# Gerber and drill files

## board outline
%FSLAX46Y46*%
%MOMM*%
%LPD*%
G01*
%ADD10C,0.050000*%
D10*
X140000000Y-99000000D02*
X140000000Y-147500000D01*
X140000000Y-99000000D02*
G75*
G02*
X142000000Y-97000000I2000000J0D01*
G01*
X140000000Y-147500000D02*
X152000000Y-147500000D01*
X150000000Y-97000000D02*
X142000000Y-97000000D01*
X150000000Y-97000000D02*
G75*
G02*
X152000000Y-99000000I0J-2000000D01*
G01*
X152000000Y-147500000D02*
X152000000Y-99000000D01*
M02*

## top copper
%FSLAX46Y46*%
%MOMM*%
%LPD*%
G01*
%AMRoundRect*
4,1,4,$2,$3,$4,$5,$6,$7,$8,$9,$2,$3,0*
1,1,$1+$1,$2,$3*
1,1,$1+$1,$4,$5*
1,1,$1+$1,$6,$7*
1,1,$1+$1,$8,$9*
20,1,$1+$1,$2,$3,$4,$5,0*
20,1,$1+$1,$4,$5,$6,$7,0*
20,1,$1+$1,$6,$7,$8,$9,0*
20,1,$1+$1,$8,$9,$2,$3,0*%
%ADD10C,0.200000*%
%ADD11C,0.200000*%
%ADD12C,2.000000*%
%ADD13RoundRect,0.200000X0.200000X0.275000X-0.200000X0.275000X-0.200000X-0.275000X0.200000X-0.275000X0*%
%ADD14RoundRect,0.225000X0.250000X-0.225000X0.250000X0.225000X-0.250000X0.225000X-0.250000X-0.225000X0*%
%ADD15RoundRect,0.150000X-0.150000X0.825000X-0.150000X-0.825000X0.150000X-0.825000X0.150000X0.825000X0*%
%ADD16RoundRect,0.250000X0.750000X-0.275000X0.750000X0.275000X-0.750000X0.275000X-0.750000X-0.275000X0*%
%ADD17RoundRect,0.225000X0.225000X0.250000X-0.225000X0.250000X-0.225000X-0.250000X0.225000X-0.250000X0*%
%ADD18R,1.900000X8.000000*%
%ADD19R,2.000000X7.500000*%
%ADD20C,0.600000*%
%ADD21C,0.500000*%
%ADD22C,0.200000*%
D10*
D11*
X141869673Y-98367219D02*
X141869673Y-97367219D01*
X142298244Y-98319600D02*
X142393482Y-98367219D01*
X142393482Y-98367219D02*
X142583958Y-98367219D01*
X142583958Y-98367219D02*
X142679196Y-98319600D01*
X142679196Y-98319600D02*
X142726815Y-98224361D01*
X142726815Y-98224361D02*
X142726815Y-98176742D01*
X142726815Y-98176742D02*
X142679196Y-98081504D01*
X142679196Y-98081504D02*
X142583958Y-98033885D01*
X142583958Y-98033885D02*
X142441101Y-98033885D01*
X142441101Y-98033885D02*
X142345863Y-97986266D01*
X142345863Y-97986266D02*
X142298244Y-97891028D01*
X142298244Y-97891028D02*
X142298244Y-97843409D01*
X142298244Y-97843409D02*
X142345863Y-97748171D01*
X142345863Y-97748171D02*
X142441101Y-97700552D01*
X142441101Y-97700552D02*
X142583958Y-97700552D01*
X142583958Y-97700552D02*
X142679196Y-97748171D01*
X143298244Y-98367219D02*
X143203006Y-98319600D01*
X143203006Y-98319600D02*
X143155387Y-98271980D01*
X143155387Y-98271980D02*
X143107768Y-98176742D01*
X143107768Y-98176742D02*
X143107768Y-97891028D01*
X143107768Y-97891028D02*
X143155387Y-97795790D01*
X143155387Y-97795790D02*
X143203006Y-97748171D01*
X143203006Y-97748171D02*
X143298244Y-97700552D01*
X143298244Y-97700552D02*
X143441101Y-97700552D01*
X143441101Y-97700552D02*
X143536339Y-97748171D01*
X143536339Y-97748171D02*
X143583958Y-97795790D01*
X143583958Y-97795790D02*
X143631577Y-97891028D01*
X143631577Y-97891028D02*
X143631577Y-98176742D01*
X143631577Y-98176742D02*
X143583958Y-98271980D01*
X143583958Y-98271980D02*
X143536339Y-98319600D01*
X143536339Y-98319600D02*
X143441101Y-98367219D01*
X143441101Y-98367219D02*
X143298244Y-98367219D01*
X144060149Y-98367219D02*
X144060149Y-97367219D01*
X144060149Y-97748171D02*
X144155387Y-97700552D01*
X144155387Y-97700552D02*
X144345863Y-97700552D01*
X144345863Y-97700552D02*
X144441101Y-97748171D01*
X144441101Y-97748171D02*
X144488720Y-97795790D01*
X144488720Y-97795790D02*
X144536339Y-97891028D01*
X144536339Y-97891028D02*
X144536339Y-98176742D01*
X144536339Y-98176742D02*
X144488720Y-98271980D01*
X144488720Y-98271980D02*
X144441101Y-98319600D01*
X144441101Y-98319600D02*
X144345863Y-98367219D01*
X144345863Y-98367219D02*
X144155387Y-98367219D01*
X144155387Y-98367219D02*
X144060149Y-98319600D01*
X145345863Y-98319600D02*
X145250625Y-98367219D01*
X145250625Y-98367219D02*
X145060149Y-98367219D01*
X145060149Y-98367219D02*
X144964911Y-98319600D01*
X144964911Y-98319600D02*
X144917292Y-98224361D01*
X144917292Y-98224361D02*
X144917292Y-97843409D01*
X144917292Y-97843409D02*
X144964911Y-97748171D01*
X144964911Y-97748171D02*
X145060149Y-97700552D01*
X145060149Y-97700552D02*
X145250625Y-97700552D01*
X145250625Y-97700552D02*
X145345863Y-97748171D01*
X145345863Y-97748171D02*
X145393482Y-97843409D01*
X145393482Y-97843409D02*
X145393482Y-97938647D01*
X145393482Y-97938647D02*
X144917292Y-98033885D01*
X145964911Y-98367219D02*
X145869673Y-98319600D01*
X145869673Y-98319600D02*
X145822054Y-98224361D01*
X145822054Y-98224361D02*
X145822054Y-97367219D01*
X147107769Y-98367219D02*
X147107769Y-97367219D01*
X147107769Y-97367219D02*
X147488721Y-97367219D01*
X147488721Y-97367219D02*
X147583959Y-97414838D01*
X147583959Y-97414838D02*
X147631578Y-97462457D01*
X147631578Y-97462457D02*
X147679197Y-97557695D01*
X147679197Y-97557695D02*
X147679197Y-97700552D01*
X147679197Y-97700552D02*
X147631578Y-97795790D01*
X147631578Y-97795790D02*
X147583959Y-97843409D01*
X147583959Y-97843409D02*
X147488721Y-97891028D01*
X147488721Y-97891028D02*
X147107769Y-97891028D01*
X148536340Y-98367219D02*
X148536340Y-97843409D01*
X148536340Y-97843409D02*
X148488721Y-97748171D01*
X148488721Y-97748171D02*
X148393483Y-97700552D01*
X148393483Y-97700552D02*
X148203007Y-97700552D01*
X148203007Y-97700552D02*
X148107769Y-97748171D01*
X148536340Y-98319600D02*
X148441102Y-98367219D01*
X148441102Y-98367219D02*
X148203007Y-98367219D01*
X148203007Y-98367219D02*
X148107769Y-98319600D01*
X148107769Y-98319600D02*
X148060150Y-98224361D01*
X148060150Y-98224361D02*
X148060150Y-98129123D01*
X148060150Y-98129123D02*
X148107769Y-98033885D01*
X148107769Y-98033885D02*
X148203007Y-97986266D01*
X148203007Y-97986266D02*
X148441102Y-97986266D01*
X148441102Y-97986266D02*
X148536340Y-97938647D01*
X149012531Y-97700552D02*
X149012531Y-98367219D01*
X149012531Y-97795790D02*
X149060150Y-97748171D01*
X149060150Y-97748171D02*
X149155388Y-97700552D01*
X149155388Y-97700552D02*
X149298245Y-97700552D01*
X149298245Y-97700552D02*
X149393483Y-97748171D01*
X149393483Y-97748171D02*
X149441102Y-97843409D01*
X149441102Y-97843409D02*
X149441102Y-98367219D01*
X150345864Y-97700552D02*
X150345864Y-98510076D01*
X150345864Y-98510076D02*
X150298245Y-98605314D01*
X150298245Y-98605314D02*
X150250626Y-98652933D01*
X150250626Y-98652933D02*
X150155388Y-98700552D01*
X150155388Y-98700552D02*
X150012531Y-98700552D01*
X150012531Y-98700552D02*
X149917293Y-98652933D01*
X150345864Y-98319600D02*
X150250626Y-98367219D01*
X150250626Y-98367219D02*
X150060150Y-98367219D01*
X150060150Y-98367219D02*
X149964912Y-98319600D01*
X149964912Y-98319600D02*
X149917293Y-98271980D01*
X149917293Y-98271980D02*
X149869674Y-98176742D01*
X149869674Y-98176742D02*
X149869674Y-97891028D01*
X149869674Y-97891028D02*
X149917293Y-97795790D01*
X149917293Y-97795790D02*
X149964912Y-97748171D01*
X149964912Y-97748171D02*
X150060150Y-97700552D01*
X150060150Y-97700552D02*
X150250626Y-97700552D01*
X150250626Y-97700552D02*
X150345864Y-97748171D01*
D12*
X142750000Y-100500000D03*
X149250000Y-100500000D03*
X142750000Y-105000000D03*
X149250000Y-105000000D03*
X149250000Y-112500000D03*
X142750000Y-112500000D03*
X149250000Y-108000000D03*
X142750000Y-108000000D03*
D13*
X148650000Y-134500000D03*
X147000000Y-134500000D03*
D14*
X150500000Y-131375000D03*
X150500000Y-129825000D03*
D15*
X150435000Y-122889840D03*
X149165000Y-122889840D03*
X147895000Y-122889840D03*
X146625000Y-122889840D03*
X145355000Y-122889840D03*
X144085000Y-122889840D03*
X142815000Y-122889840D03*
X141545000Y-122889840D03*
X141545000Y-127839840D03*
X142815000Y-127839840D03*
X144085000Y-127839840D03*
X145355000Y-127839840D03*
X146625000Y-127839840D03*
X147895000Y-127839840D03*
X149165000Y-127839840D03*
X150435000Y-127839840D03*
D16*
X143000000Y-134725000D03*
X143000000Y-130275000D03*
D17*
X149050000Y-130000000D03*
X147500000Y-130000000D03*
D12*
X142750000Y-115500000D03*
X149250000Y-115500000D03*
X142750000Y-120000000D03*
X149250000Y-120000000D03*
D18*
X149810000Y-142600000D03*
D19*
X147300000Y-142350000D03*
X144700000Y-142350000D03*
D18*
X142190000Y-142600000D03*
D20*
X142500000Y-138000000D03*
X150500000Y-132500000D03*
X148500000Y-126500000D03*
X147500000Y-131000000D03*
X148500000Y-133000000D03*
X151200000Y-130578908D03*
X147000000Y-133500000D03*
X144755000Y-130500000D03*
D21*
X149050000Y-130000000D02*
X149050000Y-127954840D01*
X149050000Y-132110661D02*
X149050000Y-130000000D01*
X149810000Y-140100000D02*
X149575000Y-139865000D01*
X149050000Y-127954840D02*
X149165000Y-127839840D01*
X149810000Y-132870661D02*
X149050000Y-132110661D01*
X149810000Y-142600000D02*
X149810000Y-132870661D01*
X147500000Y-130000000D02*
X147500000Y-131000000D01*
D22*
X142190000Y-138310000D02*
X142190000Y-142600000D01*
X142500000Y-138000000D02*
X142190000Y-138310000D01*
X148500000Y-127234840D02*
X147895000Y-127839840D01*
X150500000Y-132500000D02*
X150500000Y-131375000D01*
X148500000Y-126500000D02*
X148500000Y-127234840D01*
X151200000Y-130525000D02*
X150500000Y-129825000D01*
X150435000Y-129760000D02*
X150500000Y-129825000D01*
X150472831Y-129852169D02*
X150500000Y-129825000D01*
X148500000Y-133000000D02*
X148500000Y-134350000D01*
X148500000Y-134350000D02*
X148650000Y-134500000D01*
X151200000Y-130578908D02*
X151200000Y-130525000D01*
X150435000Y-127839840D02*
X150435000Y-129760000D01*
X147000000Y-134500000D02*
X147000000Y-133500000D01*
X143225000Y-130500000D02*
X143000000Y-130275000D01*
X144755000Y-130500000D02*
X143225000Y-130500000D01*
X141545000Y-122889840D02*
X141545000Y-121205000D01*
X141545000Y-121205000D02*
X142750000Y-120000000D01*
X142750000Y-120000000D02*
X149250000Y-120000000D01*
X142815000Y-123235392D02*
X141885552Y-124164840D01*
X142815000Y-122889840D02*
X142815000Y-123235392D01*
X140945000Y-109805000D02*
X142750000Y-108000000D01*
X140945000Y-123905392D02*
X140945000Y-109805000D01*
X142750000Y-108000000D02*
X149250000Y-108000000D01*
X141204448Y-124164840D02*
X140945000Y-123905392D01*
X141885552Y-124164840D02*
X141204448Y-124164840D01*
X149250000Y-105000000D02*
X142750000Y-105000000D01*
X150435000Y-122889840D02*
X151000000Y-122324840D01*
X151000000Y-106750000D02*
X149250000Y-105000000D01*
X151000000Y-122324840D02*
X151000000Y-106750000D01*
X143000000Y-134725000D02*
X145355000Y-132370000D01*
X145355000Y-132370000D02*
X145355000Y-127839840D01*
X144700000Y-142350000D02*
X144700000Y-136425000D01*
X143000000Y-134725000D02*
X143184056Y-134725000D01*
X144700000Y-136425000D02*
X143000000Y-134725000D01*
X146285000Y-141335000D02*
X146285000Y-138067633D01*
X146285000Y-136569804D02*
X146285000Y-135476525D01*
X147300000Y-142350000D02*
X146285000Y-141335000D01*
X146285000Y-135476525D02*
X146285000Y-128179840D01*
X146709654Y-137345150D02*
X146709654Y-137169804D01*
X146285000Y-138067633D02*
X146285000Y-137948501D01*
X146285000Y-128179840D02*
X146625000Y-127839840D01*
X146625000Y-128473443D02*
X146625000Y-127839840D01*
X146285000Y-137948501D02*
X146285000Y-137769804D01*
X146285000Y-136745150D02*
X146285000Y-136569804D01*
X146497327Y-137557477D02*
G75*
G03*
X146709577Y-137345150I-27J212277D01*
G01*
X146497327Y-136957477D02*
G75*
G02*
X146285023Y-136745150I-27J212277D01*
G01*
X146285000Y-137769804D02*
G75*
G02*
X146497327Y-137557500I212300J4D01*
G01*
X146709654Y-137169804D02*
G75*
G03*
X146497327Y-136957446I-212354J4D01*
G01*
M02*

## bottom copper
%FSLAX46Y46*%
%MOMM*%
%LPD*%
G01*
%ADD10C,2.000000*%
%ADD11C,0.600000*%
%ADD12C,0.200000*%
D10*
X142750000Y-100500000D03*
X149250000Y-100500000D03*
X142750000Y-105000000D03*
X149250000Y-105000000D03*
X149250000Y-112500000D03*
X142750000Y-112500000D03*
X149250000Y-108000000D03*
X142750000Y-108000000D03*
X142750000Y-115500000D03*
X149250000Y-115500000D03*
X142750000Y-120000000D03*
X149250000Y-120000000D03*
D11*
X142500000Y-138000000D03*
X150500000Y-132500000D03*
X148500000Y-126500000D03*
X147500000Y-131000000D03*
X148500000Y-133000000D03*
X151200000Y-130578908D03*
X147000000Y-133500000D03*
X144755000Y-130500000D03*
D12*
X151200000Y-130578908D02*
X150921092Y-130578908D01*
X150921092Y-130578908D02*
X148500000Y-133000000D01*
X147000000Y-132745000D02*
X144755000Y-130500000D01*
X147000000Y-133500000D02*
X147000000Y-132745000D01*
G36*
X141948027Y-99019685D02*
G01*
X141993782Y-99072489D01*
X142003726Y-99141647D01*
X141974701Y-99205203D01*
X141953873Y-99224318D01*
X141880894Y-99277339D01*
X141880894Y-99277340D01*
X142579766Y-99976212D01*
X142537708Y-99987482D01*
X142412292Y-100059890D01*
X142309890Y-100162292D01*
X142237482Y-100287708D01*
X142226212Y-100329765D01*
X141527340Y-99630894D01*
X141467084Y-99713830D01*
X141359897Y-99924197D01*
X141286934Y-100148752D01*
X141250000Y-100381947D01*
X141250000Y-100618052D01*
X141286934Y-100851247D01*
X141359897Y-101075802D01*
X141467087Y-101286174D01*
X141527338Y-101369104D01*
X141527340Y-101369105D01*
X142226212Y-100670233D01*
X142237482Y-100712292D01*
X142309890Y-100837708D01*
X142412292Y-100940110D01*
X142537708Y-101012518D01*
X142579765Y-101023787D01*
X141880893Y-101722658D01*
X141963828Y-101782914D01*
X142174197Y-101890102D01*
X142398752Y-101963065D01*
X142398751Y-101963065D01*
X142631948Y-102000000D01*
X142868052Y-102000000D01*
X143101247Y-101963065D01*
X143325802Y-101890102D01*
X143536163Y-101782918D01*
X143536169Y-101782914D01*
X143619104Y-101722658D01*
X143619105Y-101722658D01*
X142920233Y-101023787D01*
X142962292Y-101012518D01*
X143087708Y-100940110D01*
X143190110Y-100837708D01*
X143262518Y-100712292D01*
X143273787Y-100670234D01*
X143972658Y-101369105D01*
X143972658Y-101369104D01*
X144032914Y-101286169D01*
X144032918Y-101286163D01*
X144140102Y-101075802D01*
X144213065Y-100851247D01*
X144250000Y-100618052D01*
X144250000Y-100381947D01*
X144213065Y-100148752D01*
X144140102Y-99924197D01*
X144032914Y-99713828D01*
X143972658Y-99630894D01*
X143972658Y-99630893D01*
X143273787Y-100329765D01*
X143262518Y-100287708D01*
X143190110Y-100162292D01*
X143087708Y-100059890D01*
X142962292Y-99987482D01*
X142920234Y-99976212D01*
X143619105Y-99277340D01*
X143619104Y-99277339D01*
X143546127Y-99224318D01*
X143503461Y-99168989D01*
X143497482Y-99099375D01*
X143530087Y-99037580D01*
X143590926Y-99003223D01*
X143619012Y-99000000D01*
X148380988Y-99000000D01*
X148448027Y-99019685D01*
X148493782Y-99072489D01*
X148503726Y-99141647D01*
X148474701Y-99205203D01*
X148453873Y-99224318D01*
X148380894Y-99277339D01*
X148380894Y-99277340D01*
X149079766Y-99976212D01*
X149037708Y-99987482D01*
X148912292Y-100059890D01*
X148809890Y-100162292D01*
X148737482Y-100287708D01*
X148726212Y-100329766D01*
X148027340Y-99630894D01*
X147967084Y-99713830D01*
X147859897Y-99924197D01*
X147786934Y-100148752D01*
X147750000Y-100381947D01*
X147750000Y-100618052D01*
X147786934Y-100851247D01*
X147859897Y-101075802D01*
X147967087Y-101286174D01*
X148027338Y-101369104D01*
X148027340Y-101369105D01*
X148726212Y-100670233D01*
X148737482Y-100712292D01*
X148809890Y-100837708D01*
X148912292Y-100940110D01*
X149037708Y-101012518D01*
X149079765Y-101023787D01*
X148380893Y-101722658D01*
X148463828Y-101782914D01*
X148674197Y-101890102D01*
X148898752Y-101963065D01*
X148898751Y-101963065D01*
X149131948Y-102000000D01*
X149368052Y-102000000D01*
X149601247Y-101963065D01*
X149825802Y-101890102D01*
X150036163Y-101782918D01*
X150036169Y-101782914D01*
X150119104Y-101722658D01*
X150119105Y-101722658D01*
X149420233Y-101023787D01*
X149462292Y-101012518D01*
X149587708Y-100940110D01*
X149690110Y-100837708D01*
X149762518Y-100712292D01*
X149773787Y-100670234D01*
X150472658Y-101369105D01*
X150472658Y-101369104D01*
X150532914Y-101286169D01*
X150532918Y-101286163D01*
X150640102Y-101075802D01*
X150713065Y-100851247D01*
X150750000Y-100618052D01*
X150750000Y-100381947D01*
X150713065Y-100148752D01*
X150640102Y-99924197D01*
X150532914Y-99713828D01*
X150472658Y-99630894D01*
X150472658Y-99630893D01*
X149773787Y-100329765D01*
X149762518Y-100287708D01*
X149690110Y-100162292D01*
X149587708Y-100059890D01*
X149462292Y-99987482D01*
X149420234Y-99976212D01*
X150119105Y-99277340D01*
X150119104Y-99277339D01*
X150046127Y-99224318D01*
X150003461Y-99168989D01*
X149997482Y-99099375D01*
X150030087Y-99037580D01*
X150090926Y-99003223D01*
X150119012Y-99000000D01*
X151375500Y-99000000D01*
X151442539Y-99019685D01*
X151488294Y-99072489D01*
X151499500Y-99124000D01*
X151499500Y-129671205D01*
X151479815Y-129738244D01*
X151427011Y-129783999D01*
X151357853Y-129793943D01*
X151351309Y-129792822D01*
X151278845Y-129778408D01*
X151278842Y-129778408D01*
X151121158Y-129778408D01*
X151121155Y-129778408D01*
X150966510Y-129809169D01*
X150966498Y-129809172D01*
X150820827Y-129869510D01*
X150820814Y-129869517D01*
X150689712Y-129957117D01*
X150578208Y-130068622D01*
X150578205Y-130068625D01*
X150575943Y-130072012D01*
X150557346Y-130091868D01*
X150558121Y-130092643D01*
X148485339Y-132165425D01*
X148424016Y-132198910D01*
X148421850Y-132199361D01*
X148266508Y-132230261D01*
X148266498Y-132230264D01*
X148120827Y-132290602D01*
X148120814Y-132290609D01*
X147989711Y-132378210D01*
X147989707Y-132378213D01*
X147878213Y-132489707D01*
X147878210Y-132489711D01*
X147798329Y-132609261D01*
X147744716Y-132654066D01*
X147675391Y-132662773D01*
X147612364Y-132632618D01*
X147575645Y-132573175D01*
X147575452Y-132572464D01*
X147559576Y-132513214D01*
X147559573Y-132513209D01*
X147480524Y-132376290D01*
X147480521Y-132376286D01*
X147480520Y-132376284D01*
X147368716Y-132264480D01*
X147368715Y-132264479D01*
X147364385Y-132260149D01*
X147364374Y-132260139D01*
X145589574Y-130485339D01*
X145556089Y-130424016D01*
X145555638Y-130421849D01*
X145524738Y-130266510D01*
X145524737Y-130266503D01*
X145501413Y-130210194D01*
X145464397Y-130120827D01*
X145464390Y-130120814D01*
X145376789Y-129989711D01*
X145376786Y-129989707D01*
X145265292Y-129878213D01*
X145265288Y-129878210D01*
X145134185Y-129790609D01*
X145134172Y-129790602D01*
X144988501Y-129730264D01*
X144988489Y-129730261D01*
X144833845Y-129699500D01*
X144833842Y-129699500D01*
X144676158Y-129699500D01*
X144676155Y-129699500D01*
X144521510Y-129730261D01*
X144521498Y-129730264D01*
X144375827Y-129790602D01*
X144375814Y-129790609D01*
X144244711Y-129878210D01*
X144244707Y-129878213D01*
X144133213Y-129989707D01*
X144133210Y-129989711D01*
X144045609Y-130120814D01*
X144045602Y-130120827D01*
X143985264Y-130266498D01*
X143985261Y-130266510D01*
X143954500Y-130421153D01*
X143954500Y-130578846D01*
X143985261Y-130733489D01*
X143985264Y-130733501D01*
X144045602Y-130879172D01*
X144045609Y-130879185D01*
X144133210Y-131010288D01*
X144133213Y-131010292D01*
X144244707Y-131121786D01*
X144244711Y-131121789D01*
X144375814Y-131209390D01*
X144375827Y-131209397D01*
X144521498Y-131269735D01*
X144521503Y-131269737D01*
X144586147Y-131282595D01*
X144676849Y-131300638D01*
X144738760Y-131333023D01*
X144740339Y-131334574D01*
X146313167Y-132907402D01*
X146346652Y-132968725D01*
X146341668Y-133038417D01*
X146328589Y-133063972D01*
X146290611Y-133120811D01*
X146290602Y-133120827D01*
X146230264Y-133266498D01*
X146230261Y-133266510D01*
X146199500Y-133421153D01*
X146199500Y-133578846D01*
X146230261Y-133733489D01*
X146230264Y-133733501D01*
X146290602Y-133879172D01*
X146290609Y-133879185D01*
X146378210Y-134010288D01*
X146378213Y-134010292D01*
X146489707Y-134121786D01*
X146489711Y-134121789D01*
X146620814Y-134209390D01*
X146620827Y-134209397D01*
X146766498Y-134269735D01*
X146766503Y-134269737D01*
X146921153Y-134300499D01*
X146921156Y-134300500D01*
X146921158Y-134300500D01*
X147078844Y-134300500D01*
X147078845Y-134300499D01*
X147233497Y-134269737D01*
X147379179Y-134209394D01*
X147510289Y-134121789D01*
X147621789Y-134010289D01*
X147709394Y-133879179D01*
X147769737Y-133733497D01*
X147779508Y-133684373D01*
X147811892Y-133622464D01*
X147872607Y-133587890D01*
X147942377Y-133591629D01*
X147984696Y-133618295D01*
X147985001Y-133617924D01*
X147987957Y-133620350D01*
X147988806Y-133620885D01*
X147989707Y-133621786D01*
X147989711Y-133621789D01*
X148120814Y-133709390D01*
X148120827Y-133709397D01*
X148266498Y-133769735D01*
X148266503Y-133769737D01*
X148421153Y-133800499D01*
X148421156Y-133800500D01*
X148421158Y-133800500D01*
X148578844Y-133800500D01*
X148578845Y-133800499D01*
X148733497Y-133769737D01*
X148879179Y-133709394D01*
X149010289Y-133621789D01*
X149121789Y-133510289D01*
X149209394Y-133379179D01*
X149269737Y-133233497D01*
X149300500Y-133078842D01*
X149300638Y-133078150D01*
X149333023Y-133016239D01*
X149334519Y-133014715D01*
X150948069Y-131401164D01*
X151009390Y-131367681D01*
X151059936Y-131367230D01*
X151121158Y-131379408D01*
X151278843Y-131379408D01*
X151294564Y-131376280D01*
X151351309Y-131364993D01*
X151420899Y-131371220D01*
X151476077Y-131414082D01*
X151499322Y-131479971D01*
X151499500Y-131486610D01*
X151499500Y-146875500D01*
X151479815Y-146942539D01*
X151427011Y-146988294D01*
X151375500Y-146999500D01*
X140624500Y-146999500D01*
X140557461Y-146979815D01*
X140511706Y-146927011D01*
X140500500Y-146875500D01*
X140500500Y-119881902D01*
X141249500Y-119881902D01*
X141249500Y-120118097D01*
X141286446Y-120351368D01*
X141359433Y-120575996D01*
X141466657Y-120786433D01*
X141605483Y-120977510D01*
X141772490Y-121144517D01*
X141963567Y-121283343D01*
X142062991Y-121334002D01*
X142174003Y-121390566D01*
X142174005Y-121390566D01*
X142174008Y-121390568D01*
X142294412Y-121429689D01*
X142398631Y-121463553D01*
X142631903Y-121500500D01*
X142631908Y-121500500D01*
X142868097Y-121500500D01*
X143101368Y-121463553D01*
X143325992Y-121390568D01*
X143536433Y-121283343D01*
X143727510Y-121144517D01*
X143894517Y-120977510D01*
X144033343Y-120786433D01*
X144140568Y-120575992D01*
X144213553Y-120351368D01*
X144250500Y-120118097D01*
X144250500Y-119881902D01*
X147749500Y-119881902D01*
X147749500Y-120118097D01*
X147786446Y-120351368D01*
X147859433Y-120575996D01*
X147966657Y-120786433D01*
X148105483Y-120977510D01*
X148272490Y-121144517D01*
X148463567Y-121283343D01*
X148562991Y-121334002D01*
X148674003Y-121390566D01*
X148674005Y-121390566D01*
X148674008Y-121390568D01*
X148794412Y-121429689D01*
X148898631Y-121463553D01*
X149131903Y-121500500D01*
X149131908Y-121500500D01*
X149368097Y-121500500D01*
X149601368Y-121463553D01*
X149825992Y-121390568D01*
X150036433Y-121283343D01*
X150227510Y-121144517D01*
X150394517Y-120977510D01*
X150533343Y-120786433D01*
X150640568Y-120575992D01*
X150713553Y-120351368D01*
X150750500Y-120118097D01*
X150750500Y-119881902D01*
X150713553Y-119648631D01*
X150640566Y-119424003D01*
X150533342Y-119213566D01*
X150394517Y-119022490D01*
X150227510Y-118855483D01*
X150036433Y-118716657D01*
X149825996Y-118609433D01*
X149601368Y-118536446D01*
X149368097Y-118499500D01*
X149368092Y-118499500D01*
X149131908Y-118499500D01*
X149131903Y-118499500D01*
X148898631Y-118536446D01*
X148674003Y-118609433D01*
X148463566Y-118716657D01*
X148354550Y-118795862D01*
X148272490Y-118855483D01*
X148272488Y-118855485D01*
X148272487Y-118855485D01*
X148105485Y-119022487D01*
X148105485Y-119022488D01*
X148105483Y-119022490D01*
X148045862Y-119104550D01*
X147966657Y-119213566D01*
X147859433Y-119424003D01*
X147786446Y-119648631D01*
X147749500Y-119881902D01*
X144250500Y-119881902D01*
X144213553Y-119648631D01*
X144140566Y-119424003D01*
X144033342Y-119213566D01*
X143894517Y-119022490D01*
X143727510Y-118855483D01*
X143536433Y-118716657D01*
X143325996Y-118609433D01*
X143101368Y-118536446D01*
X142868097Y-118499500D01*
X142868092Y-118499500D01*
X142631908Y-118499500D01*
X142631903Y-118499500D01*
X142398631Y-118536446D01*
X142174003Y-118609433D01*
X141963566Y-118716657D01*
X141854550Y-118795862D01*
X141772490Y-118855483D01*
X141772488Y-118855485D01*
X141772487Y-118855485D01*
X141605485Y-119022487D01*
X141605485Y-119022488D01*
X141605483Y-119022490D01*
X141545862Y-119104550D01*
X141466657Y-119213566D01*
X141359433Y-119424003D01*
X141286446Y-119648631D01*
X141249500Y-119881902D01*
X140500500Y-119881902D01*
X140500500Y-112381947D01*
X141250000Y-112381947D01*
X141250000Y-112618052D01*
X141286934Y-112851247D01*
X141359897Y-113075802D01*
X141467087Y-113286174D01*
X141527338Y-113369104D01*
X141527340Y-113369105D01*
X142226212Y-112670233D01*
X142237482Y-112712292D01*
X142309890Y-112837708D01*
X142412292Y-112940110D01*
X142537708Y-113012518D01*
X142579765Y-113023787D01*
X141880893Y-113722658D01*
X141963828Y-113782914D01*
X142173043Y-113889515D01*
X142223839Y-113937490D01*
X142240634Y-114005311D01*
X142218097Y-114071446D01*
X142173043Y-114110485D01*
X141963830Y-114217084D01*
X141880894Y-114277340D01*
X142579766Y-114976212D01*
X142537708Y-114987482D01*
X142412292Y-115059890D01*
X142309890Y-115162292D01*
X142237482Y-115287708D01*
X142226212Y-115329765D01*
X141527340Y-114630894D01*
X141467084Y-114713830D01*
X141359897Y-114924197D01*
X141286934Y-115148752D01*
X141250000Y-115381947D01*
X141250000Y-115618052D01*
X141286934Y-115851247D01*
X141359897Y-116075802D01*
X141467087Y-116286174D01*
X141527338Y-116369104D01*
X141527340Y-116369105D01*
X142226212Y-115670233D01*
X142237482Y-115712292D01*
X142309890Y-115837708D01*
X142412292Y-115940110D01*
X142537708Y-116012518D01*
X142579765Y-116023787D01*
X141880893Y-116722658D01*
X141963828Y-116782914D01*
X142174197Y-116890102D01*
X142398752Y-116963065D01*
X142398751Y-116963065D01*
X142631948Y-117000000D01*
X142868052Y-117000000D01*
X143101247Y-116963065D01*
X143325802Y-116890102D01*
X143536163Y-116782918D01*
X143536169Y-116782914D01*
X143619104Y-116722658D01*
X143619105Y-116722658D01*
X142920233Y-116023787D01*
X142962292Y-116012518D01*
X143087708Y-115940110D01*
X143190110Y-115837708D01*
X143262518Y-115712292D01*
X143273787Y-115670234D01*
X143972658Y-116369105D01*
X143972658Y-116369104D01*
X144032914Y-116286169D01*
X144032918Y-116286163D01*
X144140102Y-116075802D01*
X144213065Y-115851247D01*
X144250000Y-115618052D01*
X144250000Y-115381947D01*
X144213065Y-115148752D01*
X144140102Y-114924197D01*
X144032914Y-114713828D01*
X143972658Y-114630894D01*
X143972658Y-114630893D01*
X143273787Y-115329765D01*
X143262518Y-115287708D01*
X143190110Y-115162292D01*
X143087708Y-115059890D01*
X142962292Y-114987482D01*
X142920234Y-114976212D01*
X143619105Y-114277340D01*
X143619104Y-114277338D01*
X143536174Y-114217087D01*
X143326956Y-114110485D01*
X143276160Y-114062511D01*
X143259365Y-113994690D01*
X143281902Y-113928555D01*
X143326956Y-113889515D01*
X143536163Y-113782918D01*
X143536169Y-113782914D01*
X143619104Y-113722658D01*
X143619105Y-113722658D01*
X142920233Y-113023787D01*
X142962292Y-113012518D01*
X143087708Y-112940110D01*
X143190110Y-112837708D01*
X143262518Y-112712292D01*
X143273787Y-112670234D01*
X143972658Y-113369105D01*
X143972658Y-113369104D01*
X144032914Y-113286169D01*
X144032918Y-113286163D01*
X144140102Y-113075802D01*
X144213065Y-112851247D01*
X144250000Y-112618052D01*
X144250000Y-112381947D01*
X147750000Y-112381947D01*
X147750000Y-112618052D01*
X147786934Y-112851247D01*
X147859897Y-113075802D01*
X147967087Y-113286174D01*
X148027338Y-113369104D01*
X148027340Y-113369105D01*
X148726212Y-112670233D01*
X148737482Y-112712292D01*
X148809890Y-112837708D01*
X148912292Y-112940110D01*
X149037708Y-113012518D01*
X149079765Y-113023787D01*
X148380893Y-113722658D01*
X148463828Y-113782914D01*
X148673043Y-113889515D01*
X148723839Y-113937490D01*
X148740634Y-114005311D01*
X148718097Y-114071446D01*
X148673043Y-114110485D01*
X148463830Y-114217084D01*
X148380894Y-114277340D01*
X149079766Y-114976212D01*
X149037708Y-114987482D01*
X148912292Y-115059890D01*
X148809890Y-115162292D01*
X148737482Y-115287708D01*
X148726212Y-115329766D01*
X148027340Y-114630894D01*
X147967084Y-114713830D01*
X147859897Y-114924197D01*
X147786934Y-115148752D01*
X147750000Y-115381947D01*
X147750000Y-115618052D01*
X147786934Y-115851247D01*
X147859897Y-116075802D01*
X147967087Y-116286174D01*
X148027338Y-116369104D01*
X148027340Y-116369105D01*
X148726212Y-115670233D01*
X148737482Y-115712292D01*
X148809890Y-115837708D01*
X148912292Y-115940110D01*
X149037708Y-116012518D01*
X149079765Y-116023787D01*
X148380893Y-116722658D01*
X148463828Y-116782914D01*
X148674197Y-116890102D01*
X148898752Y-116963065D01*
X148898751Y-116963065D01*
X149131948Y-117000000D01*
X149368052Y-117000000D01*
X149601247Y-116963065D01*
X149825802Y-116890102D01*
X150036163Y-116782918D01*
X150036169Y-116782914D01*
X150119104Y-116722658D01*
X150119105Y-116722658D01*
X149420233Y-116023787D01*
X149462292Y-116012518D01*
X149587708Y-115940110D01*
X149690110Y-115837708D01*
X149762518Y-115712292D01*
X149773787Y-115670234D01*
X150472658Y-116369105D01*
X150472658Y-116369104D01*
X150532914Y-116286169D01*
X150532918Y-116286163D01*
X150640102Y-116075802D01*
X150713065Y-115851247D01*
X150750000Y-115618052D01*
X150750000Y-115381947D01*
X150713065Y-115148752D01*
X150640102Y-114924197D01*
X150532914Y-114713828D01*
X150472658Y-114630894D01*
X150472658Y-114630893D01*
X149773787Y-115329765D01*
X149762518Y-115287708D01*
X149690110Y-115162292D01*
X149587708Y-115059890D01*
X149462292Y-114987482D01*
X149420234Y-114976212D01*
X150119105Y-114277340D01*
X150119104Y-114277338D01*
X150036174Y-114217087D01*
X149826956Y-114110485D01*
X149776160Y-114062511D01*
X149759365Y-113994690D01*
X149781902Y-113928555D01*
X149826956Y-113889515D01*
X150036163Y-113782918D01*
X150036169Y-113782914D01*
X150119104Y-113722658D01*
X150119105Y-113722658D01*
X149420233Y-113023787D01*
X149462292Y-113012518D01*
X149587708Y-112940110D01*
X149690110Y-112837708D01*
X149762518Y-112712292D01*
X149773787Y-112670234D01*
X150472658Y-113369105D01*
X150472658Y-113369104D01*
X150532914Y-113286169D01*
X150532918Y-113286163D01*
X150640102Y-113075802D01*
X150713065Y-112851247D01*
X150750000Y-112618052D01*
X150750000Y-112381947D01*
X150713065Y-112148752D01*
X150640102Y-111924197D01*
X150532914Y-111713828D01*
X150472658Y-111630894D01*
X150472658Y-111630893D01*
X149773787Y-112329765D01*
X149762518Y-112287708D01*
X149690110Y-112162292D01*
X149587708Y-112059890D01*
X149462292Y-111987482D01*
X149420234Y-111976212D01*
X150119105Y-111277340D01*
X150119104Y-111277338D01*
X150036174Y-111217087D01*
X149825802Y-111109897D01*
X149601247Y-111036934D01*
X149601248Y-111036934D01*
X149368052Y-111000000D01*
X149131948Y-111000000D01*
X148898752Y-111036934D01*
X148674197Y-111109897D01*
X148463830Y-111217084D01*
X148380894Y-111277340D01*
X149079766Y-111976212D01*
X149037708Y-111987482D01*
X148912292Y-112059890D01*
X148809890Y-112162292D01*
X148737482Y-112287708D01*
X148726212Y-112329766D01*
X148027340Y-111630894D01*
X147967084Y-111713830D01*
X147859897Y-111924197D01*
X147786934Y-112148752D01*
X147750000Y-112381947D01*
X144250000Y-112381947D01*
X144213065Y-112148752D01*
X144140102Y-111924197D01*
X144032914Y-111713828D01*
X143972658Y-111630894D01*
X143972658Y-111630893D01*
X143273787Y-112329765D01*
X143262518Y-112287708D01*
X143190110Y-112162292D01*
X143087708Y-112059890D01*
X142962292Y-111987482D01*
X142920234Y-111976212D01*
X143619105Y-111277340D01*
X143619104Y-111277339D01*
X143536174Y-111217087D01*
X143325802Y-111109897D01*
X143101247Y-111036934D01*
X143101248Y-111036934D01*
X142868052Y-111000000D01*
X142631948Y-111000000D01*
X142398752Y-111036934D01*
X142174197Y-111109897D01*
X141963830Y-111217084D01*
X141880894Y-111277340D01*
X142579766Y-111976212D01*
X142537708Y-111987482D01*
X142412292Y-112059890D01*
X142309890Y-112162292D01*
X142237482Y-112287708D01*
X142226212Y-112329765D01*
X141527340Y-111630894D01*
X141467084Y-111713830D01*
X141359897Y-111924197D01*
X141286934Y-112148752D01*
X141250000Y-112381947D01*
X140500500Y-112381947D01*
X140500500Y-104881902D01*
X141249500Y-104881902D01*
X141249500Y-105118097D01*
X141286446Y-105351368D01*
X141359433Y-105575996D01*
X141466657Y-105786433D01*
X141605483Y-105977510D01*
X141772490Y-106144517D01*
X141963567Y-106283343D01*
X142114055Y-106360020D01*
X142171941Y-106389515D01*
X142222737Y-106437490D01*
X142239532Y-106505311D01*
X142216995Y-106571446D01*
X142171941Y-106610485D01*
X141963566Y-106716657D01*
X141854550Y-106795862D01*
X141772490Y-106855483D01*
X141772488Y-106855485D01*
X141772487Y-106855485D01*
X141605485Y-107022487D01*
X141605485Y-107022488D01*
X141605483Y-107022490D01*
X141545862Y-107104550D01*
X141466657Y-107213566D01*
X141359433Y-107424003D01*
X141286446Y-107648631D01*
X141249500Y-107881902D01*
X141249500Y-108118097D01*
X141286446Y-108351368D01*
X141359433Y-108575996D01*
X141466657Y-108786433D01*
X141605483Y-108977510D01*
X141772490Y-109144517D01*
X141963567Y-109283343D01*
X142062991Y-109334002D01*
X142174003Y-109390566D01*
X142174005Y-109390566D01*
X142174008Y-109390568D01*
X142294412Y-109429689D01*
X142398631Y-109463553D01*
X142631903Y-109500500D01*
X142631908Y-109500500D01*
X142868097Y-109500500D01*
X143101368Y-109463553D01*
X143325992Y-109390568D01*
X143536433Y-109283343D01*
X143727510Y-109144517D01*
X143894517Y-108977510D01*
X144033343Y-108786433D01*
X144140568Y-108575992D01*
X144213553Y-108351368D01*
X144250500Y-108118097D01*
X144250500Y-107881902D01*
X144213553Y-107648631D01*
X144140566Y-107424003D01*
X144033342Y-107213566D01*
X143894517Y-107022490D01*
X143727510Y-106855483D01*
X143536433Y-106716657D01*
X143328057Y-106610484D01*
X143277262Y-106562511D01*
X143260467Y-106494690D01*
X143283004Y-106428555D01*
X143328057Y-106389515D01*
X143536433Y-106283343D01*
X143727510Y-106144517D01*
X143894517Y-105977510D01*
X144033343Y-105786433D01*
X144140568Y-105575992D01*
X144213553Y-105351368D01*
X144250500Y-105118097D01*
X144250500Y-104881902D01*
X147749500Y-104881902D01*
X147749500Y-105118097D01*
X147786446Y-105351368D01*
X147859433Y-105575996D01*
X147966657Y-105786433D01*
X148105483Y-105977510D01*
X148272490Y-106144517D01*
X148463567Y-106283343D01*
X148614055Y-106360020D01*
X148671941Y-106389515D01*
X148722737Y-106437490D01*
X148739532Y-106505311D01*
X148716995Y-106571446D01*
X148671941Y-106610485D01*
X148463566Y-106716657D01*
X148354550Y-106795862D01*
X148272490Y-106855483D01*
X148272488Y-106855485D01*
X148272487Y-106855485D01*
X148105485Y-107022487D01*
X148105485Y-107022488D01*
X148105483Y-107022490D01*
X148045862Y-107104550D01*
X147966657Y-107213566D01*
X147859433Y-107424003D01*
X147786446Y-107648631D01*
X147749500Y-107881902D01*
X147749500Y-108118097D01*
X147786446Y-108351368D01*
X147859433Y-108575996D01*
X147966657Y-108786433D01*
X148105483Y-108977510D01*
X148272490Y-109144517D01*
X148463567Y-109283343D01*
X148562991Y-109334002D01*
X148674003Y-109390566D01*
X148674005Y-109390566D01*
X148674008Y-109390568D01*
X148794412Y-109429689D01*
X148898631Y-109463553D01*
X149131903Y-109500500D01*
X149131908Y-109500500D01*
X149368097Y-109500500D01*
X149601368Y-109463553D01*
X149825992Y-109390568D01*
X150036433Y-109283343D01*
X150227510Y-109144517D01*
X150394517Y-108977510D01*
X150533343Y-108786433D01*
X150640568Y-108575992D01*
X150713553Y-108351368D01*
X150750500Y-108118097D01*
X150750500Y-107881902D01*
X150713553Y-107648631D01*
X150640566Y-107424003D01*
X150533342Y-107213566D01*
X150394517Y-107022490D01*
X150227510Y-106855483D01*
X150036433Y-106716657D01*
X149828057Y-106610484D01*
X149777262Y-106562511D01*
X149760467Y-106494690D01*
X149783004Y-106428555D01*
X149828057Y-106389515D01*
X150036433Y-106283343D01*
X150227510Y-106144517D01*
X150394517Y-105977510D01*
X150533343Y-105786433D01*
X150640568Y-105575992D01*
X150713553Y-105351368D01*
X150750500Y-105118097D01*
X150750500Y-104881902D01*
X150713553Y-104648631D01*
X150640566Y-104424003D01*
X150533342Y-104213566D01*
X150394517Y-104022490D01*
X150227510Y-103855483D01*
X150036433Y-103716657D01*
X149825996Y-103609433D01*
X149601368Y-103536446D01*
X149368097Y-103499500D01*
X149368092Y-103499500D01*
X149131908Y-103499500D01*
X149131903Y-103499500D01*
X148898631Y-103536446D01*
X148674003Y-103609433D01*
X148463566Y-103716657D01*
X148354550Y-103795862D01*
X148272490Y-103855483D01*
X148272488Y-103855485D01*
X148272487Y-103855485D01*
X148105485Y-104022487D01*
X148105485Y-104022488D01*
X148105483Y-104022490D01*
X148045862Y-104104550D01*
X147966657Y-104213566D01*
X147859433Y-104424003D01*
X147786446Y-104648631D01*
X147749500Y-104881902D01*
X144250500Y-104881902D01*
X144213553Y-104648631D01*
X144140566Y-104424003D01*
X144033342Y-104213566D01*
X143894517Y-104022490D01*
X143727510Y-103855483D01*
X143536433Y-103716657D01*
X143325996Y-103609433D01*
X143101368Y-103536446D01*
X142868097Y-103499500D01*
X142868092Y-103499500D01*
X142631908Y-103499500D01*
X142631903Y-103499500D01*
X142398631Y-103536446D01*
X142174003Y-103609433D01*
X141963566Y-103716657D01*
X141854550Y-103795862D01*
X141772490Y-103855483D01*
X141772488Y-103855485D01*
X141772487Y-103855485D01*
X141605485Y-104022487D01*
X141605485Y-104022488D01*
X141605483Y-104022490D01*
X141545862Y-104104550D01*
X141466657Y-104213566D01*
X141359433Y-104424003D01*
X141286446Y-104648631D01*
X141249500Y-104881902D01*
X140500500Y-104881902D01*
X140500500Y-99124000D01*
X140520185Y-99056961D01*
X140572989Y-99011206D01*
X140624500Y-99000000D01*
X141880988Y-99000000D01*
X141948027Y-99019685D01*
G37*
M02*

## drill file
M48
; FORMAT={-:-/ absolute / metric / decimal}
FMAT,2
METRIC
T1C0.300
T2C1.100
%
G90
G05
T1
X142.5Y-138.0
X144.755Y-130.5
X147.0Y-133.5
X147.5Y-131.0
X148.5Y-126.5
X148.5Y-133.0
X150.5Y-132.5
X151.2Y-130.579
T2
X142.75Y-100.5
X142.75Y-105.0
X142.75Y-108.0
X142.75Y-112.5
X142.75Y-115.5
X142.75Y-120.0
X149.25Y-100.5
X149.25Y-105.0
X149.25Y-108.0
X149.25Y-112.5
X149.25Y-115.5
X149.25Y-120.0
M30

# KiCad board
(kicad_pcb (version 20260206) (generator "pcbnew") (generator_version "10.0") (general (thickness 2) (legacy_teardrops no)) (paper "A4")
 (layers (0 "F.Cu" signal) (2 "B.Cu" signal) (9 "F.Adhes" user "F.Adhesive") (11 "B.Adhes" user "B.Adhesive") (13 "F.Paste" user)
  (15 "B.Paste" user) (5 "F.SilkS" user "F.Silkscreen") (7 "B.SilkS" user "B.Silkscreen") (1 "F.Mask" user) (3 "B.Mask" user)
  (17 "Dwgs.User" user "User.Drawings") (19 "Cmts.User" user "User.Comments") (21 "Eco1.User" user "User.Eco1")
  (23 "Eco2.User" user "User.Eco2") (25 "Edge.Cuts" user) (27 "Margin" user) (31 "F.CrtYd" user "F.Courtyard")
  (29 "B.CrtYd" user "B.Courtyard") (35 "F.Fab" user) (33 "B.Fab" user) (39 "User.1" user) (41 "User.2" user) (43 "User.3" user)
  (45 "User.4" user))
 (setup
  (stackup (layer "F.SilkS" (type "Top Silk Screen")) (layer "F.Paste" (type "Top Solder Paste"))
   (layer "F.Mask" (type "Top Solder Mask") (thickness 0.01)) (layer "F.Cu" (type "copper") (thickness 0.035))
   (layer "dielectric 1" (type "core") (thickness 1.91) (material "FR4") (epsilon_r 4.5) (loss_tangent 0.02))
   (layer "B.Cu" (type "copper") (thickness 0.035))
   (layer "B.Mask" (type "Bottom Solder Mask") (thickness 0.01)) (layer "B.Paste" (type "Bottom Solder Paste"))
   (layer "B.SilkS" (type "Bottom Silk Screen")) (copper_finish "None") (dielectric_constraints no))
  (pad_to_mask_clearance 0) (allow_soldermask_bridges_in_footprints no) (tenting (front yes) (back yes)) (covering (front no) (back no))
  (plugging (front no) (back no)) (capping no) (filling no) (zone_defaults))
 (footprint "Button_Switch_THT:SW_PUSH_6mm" (layer "F.Cu") (at 142.75 100.5)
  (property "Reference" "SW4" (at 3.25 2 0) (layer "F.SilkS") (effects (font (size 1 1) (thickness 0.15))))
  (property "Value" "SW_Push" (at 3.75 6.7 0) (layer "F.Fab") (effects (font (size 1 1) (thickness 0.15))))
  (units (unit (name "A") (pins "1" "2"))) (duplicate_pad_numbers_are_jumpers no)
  (pad "1" thru_hole circle (at 0 0 90) (size 2 2) (drill 1.1) (layers "*.Cu" "*.Mask") (remove_unused_layers no) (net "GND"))
  (pad "1" thru_hole circle (at 6.5 0 90) (size 2 2) (drill 1.1) (layers "*.Cu" "*.Mask") (remove_unused_layers no) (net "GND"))
  (pad "2" thru_hole circle (at 0 4.5 90) (size 2 2) (drill 1.1) (layers "*.Cu" "*.Mask") (remove_unused_layers no) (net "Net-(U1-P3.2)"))
  (pad "2" thru_hole circle (at 6.5 4.5 90) (size 2 2) (drill 1.1) (layers "*.Cu" "*.Mask") (remove_unused_layers no) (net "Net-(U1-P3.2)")))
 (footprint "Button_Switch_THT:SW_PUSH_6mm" (layer "F.Cu") (at 149.25 112.5 180)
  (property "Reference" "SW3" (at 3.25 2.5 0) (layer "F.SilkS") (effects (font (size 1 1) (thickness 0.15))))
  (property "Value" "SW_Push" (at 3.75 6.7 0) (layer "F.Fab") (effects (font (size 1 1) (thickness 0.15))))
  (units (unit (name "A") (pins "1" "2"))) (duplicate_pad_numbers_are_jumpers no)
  (pad "1" thru_hole circle (at 0 0 270) (size 2 2) (drill 1.1) (layers "*.Cu" "*.Mask") (remove_unused_layers no) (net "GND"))
  (pad "1" thru_hole circle (at 6.5 0 270) (size 2 2) (drill 1.1) (layers "*.Cu" "*.Mask") (remove_unused_layers no) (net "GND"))
  (pad "2" thru_hole circle (at 0 4.5 270) (size 2 2) (drill 1.1) (layers "*.Cu" "*.Mask") (remove_unused_layers no) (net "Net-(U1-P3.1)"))
  (pad "2" thru_hole circle (at 6.5 4.5 270) (size 2 2) (drill 1.1) (layers "*.Cu" "*.Mask") (remove_unused_layers no) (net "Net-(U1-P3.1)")))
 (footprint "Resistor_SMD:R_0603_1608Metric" (layer "F.Cu") (at 147.825 134.5 180)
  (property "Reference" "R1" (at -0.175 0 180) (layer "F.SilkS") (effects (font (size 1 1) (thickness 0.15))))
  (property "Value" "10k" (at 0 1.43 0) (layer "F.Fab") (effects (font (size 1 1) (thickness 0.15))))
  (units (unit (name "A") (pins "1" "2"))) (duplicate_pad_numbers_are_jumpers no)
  (pad "1" smd roundrect (at -0.825 0 180) (size 0.8 0.95) (layers "F.Cu" "F.Mask" "F.Paste") (roundrect_rratio 0.25) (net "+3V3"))
  (pad "2" smd roundrect (at 0.825 0 180) (size 0.8 0.95) (layers "F.Cu" "F.Mask" "F.Paste") (roundrect_rratio 0.25) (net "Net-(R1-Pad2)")))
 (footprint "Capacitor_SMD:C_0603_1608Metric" (layer "F.Cu") (at 150.5 130.6 90)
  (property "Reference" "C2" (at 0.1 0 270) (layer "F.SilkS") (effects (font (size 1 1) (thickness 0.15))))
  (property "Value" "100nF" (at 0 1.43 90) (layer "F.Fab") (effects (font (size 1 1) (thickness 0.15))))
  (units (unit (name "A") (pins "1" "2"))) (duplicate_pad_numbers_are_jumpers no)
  (pad "1" smd roundrect (at -0.775 0 90) (size 0.9 0.95) (layers "F.Cu" "F.Mask" "F.Paste") (roundrect_rratio 0.25) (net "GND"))
  (pad "2" smd roundrect (at 0.775 0 90) (size 0.9 0.95) (layers "F.Cu" "F.Mask" "F.Paste") (roundrect_rratio 0.25) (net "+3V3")))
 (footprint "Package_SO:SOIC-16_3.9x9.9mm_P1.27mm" (layer "F.Cu") (at 145.99 125.36484 -90)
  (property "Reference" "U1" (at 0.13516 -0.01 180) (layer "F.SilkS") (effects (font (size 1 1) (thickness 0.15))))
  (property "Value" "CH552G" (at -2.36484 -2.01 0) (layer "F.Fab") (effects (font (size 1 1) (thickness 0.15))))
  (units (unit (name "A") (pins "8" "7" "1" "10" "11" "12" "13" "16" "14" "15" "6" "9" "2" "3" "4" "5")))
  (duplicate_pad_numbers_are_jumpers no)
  (pad "1" smd roundrect (at -2.475 -4.445 270) (size 1.95 0.6) (layers "F.Cu" "F.Mask" "F.Paste") (roundrect_rratio 0.25)
   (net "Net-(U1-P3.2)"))
  (pad "2" smd roundrect (at -2.475 -3.175 270) (size 1.95 0.6) (layers "F.Cu" "F.Mask" "F.Paste") (roundrect_rratio 0.25)
   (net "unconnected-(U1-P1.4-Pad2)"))
  (pad "3" smd roundrect (at -2.475 -1.905 270) (size 1.95 0.6) (layers "F.Cu" "F.Mask" "F.Paste") (roundrect_rratio 0.25)
   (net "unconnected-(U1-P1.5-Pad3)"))
  (pad "4" smd roundrect (at -2.475 -0.635 270) (size 1.95 0.6) (layers "F.Cu" "F.Mask" "F.Paste") (roundrect_rratio 0.25)
   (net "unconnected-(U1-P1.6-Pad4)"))
  (pad "5" smd roundrect (at -2.475 0.635 270) (size 1.95 0.6) (layers "F.Cu" "F.Mask" "F.Paste") (roundrect_rratio 0.25)
   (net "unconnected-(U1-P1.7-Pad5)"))
  (pad "6" smd roundrect (at -2.475 1.905 270) (size 1.95 0.6) (layers "F.Cu" "F.Mask" "F.Paste") (roundrect_rratio 0.25)
   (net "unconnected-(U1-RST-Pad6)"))
  (pad "7" smd roundrect (at -2.475 3.175 270) (size 1.95 0.6) (layers "F.Cu" "F.Mask" "F.Paste") (roundrect_rratio 0.25)
   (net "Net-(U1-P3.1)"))
  (pad "8" smd roundrect (at -2.475 4.445 270) (size 1.95 0.6) (layers "F.Cu" "F.Mask" "F.Paste") (roundrect_rratio 0.25)
   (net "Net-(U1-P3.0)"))
  (pad "9" smd roundrect (at 2.475 4.445 270) (size 1.95 0.6) (layers "F.Cu" "F.Mask" "F.Paste") (roundrect_rratio 0.25)
   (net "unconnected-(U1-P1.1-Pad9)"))
  (pad "10" smd roundrect (at 2.475 3.175 270) (size 1.95 0.6) (layers "F.Cu" "F.Mask" "F.Paste") (roundrect_rratio 0.25)
   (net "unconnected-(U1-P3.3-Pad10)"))
  (pad "11" smd roundrect (at 2.475 1.905 270) (size 1.95 0.6) (layers "F.Cu" "F.Mask" "F.Paste") (roundrect_rratio 0.25)
   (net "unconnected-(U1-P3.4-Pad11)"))
  (pad "12" smd roundrect (at 2.475 0.635 270) (size 1.95 0.6) (layers "F.Cu" "F.Mask" "F.Paste") (roundrect_rratio 0.25) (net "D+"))
  (pad "13" smd roundrect (at 2.475 -0.635 270) (size 1.95 0.6) (layers "F.Cu" "F.Mask" "F.Paste") (roundrect_rratio 0.25) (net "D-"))
  (pad "14" smd roundrect (at 2.475 -1.905 270) (size 1.95 0.6) (layers "F.Cu" "F.Mask" "F.Paste") (roundrect_rratio 0.25) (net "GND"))
  (pad "15" smd roundrect (at 2.475 -3.175 270) (size 1.95 0.6) (layers "F.Cu" "F.Mask" "F.Paste") (roundrect_rratio 0.25) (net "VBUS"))
  (pad "16" smd roundrect (at 2.475 -4.445 270) (size 1.95 0.6) (layers "F.Cu" "F.Mask" "F.Paste") (roundrect_rratio 0.25) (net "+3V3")))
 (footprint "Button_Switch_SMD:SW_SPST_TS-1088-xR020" (layer "F.Cu") (at 143 132.5 90)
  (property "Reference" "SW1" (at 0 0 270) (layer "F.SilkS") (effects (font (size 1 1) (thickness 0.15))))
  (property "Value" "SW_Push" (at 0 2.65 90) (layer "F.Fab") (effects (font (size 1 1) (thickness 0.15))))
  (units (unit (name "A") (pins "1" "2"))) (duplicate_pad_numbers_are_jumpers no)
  (pad "1" smd roundrect (at -2.225 0 90) (size 1.05 2) (layers "F.Cu" "F.Mask" "F.Paste") (roundrect_rratio 0.2380952381) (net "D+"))
  (pad "2" smd roundrect (at 2.225 0 90) (size 1.05 2) (layers "F.Cu" "F.Mask" "F.Paste") (roundrect_rratio 0.2380952381)
   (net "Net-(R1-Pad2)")))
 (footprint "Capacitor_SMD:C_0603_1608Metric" (layer "F.Cu") (at 148.275 130 180)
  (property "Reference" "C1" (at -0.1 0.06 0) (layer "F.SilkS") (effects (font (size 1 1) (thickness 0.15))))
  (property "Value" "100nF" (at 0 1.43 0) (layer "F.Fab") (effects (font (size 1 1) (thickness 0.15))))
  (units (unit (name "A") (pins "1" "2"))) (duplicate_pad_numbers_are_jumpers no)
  (pad "1" smd roundrect (at -0.775 0 180) (size 0.9 0.95) (layers "F.Cu" "F.Mask" "F.Paste") (roundrect_rratio 0.25) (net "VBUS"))
  (pad "2" smd roundrect (at 0.775 0 180) (size 0.9 0.95) (layers "F.Cu" "F.Mask" "F.Paste") (roundrect_rratio 0.25) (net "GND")))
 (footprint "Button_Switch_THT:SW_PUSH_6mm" (layer "F.Cu") (at 142.75 115.5)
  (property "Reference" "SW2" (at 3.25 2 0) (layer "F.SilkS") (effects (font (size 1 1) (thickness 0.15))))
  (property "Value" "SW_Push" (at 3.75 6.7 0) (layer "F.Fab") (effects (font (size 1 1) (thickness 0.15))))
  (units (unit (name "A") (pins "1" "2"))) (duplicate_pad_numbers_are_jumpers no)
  (pad "1" thru_hole circle (at 0 0 90) (size 2 2) (drill 1.1) (layers "*.Cu" "*.Mask") (remove_unused_layers no) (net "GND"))
  (pad "1" thru_hole circle (at 6.5 0 90) (size 2 2) (drill 1.1) (layers "*.Cu" "*.Mask") (remove_unused_layers no) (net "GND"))
  (pad "2" thru_hole circle (at 0 4.5 90) (size 2 2) (drill 1.1) (layers "*.Cu" "*.Mask") (remove_unused_layers no) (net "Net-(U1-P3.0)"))
  (pad "2" thru_hole circle (at 6.5 4.5 90) (size 2 2) (drill 1.1) (layers "*.Cu" "*.Mask") (remove_unused_layers no) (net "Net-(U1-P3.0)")))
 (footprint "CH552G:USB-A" (layer "F.Cu") (at 146 147.5)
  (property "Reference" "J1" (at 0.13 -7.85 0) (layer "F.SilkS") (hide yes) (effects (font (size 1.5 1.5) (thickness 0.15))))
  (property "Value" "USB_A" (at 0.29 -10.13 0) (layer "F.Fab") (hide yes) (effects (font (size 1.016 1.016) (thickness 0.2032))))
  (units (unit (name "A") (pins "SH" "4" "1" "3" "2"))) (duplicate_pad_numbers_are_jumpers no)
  (pad "1" connect rect (at 3.81 -4.9) (size 1.9 8) (layers "F.Cu" "F.Mask") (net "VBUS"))
  (pad "2" connect rect (at 1.3 -5.15) (size 2 7.5) (layers "F.Cu" "F.Mask") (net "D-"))
  (pad "3" connect rect (at -1.3 -5.15) (size 2 7.5) (layers "F.Cu" "F.Mask") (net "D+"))
  (pad "4" connect rect (at -3.81 -4.9) (size 1.9 8) (layers "F.Cu" "F.Mask") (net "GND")))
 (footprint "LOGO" (layer "B.Cu") (at 146 127 180)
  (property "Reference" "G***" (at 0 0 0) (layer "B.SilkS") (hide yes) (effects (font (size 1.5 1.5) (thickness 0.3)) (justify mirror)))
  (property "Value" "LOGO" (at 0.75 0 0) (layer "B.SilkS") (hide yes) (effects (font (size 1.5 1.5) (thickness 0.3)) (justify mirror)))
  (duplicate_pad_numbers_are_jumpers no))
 (gr_line (start 140 99) (end 140 147.5) (stroke (width 0.05) (type default)) (layer "Edge.Cuts"))
 (gr_arc (start 140 99) (mid 140.585786 97.585786) (end 142 97) (stroke (width 0.05) (type default)) (layer "Edge.Cuts"))
 (gr_line (start 140 147.5) (end 152 147.5) (stroke (width 0.05) (type default)) (layer "Edge.Cuts"))
 (gr_line (start 150 97) (end 142 97) (stroke (width 0.05) (type default)) (layer "Edge.Cuts"))
 (gr_arc (start 150 97) (mid 151.414214 97.585786) (end 152 99) (stroke (width 0.05) (type default)) (layer "Edge.Cuts"))
 (gr_line (start 152 147.5) (end 152 99) (stroke (width 0.05) (type default)) (layer "Edge.Cuts"))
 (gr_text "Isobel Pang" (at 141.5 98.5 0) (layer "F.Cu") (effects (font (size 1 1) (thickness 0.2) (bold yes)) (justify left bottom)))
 (segment (start 149.05 130) (end 149.05 127.95484) (width 0.5) (layer "F.Cu") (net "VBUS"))
 (segment (start 149.05 132.110661) (end 149.05 130) (width 0.5) (layer "F.Cu") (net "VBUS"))
 (segment (start 149.81 140.1) (end 149.575 139.865) (width 0.5) (layer "F.Cu") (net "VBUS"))
 (segment (start 149.05 127.95484) (end 149.165 127.83984) (width 0.5) (layer "F.Cu") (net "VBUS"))
 (segment (start 149.81 132.870661) (end 149.05 132.110661) (width 0.5) (layer "F.Cu") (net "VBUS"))
 (segment (start 149.81 142.6) (end 149.81 132.870661) (width 0.5) (layer "F.Cu") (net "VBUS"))
 (segment (start 147.5 130) (end 147.5 131) (width 0.5) (layer "F.Cu") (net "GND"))
 (segment (start 142.19 138.31) (end 142.19 142.6) (width 0.2) (layer "F.Cu") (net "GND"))
 (segment (start 142.5 138) (end 142.19 138.31) (width 0.2) (layer "F.Cu") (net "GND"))
 (segment (start 148.5 127.23484) (end 147.895 127.83984) (width 0.2) (layer "F.Cu") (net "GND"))
 (segment (start 150.5 132.5) (end 150.5 131.375) (width 0.2) (layer "F.Cu") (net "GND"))
 (segment (start 148.5 126.5) (end 148.5 127.23484) (width 0.2) (layer "F.Cu") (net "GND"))
 (via (at 142.5 138) (size 0.6) (drill 0.3) (layers "F.Cu" "B.Cu") (free yes) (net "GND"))
 (via (at 150.5 132.5) (size 0.6) (drill 0.3) (layers "F.Cu" "B.Cu") (free yes) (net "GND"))
 (via (at 148.5 126.5) (size 0.6) (drill 0.3) (layers "F.Cu" "B.Cu") (free yes) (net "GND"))
 (via (at 147.5 131) (size 0.6) (drill 0.3) (layers "F.Cu" "B.Cu") (free yes) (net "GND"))
 (segment (start 151.2 130.525) (end 150.5 129.825) (width 0.2) (layer "F.Cu") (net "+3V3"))
 (segment (start 150.435 129.76) (end 150.5 129.825) (width 0.2) (layer "F.Cu") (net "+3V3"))
 (segment (start 150.472831 129.852169) (end 150.5 129.825) (width 0.2) (layer "F.Cu") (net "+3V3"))
 (segment (start 148.5 133) (end 148.5 134.35) (width 0.2) (layer "F.Cu") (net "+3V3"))
 (segment (start 148.5 134.35) (end 148.65 134.5) (width 0.2) (layer "F.Cu") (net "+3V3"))
 (segment (start 151.2 130.578908) (end 151.2 130.525) (width 0.2) (layer "F.Cu") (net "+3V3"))
 (segment (start 150.435 127.83984) (end 150.435 129.76) (width 0.2) (layer "F.Cu") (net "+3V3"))
 (via (at 148.5 133) (size 0.6) (drill 0.3) (layers "F.Cu" "B.Cu") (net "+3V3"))
 (via (at 151.2 130.578908) (size 0.6) (drill 0.3) (layers "F.Cu" "B.Cu") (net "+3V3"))
 (segment (start 151.2 130.578908) (end 150.921092 130.578908) (width 0.2) (layer "B.Cu") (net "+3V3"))
 (segment (start 150.921092 130.578908) (end 148.5 133) (width 0.2) (layer "B.Cu") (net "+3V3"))
 (segment (start 147 134.5) (end 147 133.5) (width 0.2) (layer "F.Cu") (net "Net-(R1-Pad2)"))
 (segment (start 143.225 130.5) (end 143 130.275) (width 0.2) (layer "F.Cu") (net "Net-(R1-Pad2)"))
 (segment (start 144.755 130.5) (end 143.225 130.5) (width 0.2) (layer "F.Cu") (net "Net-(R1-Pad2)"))
 (via (at 147 133.5) (size 0.6) (drill 0.3) (layers "F.Cu" "B.Cu") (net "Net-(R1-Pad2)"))
 (via (at 144.755 130.5) (size 0.6) (drill 0.3) (layers "F.Cu" "B.Cu") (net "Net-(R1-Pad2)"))
 (segment (start 147 132.745) (end 144.755 130.5) (width 0.2) (layer "B.Cu") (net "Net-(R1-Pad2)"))
 (segment (start 147 133.5) (end 147 132.745) (width 0.2) (layer "B.Cu") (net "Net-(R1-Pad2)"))
 (segment (start 141.545 122.88984) (end 141.545 121.205) (width 0.2) (layer "F.Cu") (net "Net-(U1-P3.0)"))
 (segment (start 141.545 121.205) (end 142.75 120) (width 0.2) (layer "F.Cu") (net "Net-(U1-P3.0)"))
 (segment (start 142.75 120) (end 149.25 120) (width 0.2) (layer "F.Cu") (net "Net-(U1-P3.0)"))
 (segment (start 142.815 123.235392) (end 141.885552 124.16484) (width 0.2) (layer "F.Cu") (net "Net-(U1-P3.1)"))
 (segment (start 142.815 122.88984) (end 142.815 123.235392) (width 0.2) (layer "F.Cu") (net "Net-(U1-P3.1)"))
 (segment (start 140.945 109.805) (end 142.75 108) (width 0.2) (layer "F.Cu") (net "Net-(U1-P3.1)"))
 (segment (start 140.945 123.905392) (end 140.945 109.805) (width 0.2) (layer "F.Cu") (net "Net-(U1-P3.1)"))
 (segment (start 142.75 108) (end 149.25 108) (width 0.2) (layer "F.Cu") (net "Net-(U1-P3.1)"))
 (segment (start 141.204448 124.16484) (end 140.945 123.905392) (width 0.2) (layer "F.Cu") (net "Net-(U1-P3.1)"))
 (segment (start 141.885552 124.16484) (end 141.204448 124.16484) (width 0.2) (layer "F.Cu") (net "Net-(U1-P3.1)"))
 (segment (start 149.25 105) (end 142.75 105) (width 0.2) (layer "F.Cu") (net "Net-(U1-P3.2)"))
 (segment (start 150.435 122.88984) (end 151 122.32484) (width 0.2) (layer "F.Cu") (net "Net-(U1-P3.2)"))
 (segment (start 151 106.75) (end 149.25 105) (width 0.2) (layer "F.Cu") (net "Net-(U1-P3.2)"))
 (segment (start 151 122.32484) (end 151 106.75) (width 0.2) (layer "F.Cu") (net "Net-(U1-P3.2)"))
 (segment (start 143 134.725) (end 145.355 132.37) (width 0.2) (layer "F.Cu") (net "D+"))
 (segment (start 145.355 132.37) (end 145.355 127.83984) (width 0.2) (layer "F.Cu") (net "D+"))
 (segment (start 144.7 142.35) (end 144.7 136.425) (width 0.2) (layer "F.Cu") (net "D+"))
 (segment (start 143 134.725) (end 143.184056 134.725) (width 0.2) (layer "F.Cu") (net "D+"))
 (segment (start 144.7 136.425) (end 143 134.725) (width 0.2) (layer "F.Cu") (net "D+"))
 (segment (start 146.285 141.335) (end 146.285 138.067633) (width 0.2) (layer "F.Cu") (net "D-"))
 (segment (start 146.285 136.569804) (end 146.285 135.476525) (width 0.2) (layer "F.Cu") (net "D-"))
 (segment (start 147.3 142.35) (end 146.285 141.335) (width 0.2) (layer "F.Cu") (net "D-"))
 (segment (start 146.285 135.476525) (end 146.285 128.17984) (width 0.2) (layer "F.Cu") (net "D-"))
 (segment (start 146.709654 137.34515) (end 146.709654 137.169804) (width 0.2) (layer "F.Cu") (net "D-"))
 (segment (start 146.285 138.067633) (end 146.285 137.948501) (width 0.2) (layer "F.Cu") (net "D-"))
 (segment (start 146.285 128.17984) (end 146.625 127.83984) (width 0.2) (layer "F.Cu") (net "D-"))
 (segment (start 146.625 128.473443) (end 146.625 127.83984) (width 0.2) (layer "F.Cu") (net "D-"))
 (segment (start 146.285 137.948501) (end 146.285 137.769804) (width 0.2) (layer "F.Cu") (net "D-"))
 (segment (start 146.285 136.74515) (end 146.285 136.569804) (width 0.2) (layer "F.Cu") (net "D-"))
 (arc (start 146.497327 137.557477) (mid 146.647465 137.495288) (end 146.709654 137.34515) (width 0.2) (layer "F.Cu") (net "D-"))
 (arc (start 146.497327 136.957477) (mid 146.347189 136.895288) (end 146.285 136.74515) (width 0.2) (layer "F.Cu") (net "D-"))
 (arc (start 146.285 137.769804) (mid 146.347189 137.619666) (end 146.497327 137.557477) (width 0.2) (layer "F.Cu") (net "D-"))
 (arc (start 146.709654 137.169804) (mid 146.647465 137.019666) (end 146.497327 136.957477) (width 0.2) (layer "F.Cu") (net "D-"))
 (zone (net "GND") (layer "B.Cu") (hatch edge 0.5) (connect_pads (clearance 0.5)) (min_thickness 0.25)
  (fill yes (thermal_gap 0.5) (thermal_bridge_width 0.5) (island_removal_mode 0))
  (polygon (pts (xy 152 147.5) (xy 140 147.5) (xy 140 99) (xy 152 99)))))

